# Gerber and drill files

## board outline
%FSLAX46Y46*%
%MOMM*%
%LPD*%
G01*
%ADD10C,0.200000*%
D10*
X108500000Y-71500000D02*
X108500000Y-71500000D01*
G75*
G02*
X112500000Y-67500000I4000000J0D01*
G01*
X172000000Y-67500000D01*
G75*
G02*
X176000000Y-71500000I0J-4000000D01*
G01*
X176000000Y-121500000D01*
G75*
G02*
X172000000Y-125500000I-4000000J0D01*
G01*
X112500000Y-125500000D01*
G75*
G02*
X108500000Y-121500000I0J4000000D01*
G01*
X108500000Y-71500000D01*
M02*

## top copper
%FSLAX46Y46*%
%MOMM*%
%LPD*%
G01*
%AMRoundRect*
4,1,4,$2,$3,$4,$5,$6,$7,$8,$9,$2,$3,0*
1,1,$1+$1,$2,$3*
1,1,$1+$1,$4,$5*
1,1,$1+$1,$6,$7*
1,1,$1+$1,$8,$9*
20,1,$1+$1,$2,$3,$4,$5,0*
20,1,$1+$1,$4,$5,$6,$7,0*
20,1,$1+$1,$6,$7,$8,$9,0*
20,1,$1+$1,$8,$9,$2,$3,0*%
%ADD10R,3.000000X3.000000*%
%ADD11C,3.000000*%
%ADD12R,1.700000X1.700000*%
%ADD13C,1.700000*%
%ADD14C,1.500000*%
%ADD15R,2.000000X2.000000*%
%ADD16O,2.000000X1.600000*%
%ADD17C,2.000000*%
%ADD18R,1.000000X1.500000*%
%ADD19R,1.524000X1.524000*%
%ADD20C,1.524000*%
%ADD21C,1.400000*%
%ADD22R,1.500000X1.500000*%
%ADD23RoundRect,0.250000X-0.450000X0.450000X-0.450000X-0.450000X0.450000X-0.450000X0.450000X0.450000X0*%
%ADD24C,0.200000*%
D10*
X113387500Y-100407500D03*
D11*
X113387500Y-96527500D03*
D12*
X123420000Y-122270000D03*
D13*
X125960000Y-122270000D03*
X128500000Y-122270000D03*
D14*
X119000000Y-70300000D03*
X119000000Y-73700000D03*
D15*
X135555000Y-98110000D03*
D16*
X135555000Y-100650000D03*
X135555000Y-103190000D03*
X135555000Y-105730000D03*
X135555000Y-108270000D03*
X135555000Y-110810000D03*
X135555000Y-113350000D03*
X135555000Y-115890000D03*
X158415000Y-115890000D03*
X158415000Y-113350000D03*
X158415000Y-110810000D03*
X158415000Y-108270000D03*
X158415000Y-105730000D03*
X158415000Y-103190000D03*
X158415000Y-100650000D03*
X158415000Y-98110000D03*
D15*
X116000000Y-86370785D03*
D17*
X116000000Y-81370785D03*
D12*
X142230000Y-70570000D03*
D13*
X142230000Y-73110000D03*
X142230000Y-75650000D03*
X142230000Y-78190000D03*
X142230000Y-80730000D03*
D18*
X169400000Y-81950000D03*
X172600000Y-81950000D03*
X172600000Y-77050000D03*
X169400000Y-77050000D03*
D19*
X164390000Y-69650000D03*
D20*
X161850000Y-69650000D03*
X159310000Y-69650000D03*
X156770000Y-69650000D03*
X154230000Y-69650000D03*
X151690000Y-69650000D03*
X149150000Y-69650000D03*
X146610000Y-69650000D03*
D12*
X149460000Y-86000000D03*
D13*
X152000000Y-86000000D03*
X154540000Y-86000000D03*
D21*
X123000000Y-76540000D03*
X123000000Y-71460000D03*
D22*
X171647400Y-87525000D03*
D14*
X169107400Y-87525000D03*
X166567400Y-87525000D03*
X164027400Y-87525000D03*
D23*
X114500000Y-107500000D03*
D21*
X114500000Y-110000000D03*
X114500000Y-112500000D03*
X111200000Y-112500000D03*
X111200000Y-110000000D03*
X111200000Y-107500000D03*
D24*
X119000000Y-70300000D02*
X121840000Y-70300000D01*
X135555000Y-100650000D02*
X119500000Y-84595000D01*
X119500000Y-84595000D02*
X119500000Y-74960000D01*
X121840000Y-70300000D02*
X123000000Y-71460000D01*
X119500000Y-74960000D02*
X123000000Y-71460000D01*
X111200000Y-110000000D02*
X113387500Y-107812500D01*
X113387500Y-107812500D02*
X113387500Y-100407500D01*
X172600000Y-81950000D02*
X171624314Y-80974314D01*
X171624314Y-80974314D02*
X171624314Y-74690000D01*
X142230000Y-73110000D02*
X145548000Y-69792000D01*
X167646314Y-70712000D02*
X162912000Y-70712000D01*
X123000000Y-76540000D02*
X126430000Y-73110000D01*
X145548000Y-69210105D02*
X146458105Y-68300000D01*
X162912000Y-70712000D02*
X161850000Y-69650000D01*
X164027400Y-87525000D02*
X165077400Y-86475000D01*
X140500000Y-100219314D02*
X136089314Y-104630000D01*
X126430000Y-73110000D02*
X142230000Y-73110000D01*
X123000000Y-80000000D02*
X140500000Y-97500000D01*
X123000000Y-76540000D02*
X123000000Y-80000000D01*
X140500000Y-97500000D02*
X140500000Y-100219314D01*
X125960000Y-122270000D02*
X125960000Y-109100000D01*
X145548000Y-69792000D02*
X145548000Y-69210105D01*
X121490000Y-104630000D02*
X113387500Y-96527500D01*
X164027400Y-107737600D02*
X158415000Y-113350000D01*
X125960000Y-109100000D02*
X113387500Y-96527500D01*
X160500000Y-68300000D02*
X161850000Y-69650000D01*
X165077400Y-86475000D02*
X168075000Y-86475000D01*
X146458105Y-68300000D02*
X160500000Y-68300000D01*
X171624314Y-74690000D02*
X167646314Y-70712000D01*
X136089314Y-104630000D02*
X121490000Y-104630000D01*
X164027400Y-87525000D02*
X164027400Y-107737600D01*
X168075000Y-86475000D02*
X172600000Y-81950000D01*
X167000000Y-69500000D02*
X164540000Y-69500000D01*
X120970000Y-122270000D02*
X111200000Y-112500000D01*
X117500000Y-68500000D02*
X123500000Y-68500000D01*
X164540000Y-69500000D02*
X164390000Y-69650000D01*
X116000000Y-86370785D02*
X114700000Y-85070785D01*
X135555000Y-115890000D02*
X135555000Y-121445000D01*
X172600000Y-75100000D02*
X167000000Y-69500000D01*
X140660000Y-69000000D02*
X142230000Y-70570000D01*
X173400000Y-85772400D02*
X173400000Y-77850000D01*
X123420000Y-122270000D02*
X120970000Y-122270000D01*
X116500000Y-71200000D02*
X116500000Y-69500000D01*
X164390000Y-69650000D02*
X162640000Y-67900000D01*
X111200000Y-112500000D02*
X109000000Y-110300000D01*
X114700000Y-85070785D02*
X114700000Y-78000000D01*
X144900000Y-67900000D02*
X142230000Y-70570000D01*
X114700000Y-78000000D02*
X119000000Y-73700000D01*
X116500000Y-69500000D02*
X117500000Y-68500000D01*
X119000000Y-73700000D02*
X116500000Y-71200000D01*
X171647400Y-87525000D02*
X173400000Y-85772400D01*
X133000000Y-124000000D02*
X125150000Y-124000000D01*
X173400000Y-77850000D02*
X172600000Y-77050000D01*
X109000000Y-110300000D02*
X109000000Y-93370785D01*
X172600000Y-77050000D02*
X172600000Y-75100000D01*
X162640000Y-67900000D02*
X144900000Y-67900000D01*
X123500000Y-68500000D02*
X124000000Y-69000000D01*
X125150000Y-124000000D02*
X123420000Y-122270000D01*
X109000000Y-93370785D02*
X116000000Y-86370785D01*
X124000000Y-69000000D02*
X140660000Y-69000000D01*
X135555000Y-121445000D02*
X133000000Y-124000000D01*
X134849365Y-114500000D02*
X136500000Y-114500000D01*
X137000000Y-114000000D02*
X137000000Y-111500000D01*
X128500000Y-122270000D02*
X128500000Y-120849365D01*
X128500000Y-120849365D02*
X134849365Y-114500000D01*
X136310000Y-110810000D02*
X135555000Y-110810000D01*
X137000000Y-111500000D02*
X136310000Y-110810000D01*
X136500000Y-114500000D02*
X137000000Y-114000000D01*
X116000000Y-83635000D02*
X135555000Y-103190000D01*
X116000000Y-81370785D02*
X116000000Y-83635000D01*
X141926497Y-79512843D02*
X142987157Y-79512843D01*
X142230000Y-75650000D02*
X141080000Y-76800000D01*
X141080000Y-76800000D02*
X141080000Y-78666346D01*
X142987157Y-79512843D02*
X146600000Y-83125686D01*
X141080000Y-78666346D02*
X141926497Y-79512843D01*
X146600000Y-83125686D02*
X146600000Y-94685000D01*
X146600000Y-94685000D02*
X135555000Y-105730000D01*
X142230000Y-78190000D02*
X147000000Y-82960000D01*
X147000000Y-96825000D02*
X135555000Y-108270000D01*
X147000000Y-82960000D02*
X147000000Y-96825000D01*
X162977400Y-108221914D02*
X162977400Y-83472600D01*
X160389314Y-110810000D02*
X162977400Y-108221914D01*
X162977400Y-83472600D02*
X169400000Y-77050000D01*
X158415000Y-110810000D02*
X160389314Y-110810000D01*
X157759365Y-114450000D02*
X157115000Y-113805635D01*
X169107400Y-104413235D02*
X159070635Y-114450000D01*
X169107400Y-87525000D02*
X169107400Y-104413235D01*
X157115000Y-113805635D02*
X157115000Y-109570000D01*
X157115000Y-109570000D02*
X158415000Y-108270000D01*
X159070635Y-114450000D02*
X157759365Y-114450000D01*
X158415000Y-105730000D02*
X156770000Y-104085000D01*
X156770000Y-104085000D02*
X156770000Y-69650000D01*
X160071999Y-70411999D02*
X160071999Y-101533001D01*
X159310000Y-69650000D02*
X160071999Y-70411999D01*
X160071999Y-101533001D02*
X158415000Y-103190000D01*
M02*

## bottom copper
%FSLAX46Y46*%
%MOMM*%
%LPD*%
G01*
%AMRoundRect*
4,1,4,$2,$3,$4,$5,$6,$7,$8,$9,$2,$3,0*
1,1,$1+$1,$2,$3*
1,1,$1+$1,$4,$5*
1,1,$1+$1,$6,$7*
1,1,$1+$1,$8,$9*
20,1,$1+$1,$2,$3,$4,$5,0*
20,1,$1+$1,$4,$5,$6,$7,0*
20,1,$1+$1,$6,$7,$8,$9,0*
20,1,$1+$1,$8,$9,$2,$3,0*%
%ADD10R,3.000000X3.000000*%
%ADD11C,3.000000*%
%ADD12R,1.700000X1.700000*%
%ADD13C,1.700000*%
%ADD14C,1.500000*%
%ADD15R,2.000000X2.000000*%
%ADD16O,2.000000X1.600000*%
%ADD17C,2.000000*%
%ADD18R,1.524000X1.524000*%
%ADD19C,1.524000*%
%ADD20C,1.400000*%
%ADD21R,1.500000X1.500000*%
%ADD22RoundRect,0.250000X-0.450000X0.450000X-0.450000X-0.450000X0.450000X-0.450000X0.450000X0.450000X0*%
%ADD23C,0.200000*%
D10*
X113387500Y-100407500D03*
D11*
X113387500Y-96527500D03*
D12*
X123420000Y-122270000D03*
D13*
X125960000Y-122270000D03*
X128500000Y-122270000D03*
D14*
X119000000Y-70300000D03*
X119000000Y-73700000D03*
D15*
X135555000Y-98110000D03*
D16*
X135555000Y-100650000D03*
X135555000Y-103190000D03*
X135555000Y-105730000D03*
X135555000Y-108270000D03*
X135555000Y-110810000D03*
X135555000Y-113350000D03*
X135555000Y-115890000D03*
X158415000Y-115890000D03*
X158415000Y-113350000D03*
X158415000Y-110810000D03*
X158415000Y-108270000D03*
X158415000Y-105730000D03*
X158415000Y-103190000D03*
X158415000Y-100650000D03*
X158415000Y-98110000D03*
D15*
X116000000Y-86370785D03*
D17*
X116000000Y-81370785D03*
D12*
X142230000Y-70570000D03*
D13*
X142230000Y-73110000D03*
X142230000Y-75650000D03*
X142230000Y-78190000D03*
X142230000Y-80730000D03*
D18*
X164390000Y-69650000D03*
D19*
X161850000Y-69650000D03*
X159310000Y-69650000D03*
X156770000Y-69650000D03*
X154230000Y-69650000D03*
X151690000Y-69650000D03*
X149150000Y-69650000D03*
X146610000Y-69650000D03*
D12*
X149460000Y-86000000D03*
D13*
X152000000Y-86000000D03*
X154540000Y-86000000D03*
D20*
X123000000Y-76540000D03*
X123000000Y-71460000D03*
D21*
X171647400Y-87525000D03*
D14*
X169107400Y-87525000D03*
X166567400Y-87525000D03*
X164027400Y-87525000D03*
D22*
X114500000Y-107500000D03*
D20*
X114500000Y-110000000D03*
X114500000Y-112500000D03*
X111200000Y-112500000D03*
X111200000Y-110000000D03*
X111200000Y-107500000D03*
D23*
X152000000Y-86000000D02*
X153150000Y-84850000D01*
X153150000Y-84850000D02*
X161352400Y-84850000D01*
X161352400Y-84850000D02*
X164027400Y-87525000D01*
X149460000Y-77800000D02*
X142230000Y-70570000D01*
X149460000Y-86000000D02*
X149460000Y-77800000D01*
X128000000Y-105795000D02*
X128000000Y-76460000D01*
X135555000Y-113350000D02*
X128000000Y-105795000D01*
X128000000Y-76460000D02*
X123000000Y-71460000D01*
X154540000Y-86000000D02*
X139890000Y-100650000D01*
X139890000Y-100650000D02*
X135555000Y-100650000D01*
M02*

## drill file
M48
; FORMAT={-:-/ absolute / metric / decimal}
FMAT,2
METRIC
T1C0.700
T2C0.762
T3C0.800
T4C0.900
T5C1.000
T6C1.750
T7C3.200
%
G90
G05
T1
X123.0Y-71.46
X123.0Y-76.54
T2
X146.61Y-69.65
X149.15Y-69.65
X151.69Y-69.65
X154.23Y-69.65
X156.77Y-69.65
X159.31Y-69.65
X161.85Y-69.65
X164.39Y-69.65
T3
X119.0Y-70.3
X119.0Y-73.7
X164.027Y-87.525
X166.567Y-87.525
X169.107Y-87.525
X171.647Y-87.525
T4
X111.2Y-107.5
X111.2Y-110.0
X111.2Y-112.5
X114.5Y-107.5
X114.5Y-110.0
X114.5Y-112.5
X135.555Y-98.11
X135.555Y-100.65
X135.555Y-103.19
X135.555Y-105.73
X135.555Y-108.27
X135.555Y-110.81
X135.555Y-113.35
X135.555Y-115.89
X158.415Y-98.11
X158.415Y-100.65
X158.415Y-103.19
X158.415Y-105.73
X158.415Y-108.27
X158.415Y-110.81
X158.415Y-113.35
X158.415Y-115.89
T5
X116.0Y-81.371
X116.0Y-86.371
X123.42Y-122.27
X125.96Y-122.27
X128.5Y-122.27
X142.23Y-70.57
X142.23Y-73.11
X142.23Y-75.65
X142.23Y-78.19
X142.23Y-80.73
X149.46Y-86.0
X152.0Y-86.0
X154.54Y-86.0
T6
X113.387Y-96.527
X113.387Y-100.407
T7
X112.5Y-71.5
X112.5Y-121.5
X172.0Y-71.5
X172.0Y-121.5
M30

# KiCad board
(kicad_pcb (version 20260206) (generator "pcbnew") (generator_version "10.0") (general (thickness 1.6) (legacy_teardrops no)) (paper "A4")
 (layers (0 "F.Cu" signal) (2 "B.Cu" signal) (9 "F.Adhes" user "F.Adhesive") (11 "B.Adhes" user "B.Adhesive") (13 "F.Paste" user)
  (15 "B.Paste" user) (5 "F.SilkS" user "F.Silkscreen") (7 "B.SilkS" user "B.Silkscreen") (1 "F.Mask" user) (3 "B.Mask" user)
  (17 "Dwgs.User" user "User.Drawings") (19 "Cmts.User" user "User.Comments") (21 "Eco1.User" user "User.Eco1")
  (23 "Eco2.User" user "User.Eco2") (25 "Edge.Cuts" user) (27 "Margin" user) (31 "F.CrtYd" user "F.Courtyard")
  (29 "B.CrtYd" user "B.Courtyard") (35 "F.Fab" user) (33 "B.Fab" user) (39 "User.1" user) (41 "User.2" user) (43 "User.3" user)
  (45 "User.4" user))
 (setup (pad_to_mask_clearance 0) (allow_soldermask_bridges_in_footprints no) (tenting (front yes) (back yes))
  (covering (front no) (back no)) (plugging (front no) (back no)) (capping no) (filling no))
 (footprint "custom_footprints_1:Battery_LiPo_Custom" (layer "F.Cu") (at 120.9375 98.0575 90)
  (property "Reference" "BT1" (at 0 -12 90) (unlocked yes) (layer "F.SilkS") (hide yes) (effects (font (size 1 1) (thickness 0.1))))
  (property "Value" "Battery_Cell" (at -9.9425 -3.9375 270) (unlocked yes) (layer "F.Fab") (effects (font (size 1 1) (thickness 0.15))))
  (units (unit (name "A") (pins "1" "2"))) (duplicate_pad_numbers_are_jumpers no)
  (pad "1" thru_hole rect (at -2.35 -7.55 90) (size 3 3) (drill 1.75) (layers "*.Cu" "*.Mask") (remove_unused_layers no) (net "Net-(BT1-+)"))
  (pad "2" thru_hole circle (at 1.53 -7.55 90) (size 3 3) (drill 1.75) (layers "*.Cu" "*.Mask") (remove_unused_layers no)
   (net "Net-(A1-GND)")))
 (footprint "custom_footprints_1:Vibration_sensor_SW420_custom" (layer "F.Cu") (at 130.27 122 90)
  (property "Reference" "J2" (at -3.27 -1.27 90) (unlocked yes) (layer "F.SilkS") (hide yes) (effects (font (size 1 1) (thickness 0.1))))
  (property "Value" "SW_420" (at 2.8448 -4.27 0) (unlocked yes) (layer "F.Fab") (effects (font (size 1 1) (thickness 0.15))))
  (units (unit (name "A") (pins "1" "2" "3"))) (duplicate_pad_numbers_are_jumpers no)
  (pad "1" thru_hole rect (at -0.27 -6.85 90) (size 1.7 1.7) (drill 1) (layers "*.Cu" "*.Mask") (remove_unused_layers no)
   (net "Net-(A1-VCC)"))
  (pad "2" thru_hole circle (at -0.27 -4.31 90) (size 1.7 1.7) (drill 1) (layers "*.Cu" "*.Mask") (remove_unused_layers no)
   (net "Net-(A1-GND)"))
  (pad "3" thru_hole circle (at -0.27 -1.77 90) (size 1.7 1.7) (drill 1) (layers "*.Cu" "*.Mask") (remove_unused_layers no)
   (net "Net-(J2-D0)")))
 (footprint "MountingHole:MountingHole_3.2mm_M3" (layer "F.Cu") (at 112.5 71.5 180)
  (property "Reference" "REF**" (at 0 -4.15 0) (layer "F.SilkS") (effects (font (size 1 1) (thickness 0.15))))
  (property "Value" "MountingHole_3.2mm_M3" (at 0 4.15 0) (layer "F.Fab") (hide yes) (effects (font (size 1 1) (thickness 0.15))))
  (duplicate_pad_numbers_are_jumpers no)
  (pad "" np_thru_hole circle (at 0 0 180) (size 3.2 3.2) (drill 3.2) (layers "*.Cu" "*.Mask")))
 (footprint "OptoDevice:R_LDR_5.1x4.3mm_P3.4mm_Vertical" (layer "F.Cu") (at 119 70.3 -90)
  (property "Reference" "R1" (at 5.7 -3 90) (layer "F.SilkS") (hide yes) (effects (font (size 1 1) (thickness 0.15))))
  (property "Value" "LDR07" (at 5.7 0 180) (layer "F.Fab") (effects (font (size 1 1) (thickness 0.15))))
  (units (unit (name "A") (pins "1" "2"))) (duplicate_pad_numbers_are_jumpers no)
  (pad "1" thru_hole circle (at 0 0 270) (size 1.5 1.5) (drill 0.8) (layers "*.Cu" "*.Mask") (remove_unused_layers no)
   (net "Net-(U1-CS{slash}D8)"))
  (pad "2" thru_hole circle (at 3.4 0 270) (size 1.5 1.5) (drill 0.8) (layers "*.Cu" "*.Mask") (remove_unused_layers no)
   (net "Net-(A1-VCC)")))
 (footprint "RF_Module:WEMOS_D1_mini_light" (layer "F.Cu") (at 135.555 98.11)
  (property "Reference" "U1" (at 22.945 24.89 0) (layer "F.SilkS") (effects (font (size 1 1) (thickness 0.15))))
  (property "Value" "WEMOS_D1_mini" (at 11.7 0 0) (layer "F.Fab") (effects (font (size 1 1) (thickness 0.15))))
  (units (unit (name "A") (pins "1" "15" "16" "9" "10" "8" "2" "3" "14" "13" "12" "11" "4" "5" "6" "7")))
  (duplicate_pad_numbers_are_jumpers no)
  (pad "1" thru_hole rect (at 0 0) (size 2 2) (drill 0.9) (layers "*.Cu" "*.Mask") (remove_unused_layers no)
   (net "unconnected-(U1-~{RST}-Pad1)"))
  (pad "2" thru_hole oval (at 0 2.54) (size 2 1.6) (drill 0.9) (layers "*.Cu" "*.Mask") (remove_unused_layers no) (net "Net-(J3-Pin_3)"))
  (pad "3" thru_hole oval (at 0 5.08) (size 2 1.6) (drill 0.9) (layers "*.Cu" "*.Mask") (remove_unused_layers no) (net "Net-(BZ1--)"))
  (pad "4" thru_hole oval (at 0 7.62) (size 2 1.6) (drill 0.9) (layers "*.Cu" "*.Mask") (remove_unused_layers no) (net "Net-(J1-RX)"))
  (pad "5" thru_hole oval (at 0 10.16) (size 2 1.6) (drill 0.9) (layers "*.Cu" "*.Mask") (remove_unused_layers no) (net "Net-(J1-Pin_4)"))
  (pad "6" thru_hole oval (at 0 12.7) (size 2 1.6) (drill 0.9) (layers "*.Cu" "*.Mask") (remove_unused_layers no) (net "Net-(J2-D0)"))
  (pad "7" thru_hole oval (at 0 15.24) (size 2 1.6) (drill 0.9) (layers "*.Cu" "*.Mask") (remove_unused_layers no)
   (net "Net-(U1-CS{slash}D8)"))
  (pad "8" thru_hole oval (at 0 17.78) (size 2 1.6) (drill 0.9) (layers "*.Cu" "*.Mask") (remove_unused_layers no) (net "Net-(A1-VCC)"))
  (pad "9" thru_hole oval (at 22.86 17.78) (size 2 1.6) (drill 0.9) (layers "*.Cu" "*.Mask") (remove_unused_layers no)
   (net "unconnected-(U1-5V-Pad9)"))
  (pad "10" thru_hole oval (at 22.86 15.24) (size 2 1.6) (drill 0.9) (layers "*.Cu" "*.Mask") (remove_unused_layers no) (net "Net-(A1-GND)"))
  (pad "11" thru_hole oval (at 22.86 12.7) (size 2 1.6) (drill 0.9) (layers "*.Cu" "*.Mask") (remove_unused_layers no) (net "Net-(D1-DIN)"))
  (pad "12" thru_hole oval (at 22.86 10.16) (size 2 1.6) (drill 0.9) (layers "*.Cu" "*.Mask") (remove_unused_layers no) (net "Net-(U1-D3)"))
  (pad "13" thru_hole oval (at 22.86 7.62) (size 2 1.6) (drill 0.9) (layers "*.Cu" "*.Mask") (remove_unused_layers no) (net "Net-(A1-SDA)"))
  (pad "14" thru_hole oval (at 22.86 5.08) (size 2 1.6) (drill 0.9) (layers "*.Cu" "*.Mask") (remove_unused_layers no) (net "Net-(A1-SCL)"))
  (pad "15" thru_hole oval (at 22.86 2.54) (size 2 1.6) (drill 0.9) (layers "*.Cu" "*.Mask") (remove_unused_layers no)
   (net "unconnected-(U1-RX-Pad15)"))
  (pad "16" thru_hole oval (at 22.86 0) (size 2 1.6) (drill 0.9) (layers "*.Cu" "*.Mask") (remove_unused_layers no)
   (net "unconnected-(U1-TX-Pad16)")))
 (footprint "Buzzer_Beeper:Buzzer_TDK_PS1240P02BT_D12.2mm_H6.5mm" (layer "F.Cu") (at 116 86.370785 90)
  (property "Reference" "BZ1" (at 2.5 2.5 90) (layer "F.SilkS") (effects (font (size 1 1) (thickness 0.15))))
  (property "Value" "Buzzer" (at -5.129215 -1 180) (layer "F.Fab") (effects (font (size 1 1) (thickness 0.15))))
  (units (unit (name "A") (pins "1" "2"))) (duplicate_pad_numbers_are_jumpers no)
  (pad "1" thru_hole rect (at 0 0 90) (size 2 2) (drill 1) (layers "*.Cu" "*.Mask") (remove_unused_layers no) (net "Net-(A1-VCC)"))
  (pad "2" thru_hole circle (at 5 0 90) (size 2 2) (drill 1) (layers "*.Cu" "*.Mask") (remove_unused_layers no) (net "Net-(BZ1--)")))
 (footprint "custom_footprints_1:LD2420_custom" (layer "F.Cu") (at 134.73 77.57)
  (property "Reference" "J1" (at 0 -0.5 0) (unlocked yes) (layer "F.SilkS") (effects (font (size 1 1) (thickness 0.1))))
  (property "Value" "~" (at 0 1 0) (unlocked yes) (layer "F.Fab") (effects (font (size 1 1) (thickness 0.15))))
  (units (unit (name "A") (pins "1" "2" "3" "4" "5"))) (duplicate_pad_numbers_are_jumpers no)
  (pad "1" thru_hole rect (at 7.5 -7) (size 1.7 1.7) (drill 1) (layers "*.Cu" "*.Mask") (remove_unused_layers no) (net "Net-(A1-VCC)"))
  (pad "2" thru_hole circle (at 7.5 -4.46) (size 1.7 1.7) (drill 1) (layers "*.Cu" "*.Mask") (remove_unused_layers no) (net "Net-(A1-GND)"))
  (pad "3" thru_hole circle (at 7.5 -1.92) (size 1.7 1.7) (drill 1) (layers "*.Cu" "*.Mask") (remove_unused_layers no) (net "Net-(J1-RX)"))
  (pad "4" thru_hole circle (at 7.5 0.62) (size 1.7 1.7) (drill 1) (layers "*.Cu" "*.Mask") (remove_unused_layers no) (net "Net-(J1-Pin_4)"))
  (pad "5" thru_hole circle (at 7.5 3.16) (size 1.7 1.7) (drill 1) (layers "*.Cu" "*.Mask") (remove_unused_layers no)
   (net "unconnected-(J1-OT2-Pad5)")))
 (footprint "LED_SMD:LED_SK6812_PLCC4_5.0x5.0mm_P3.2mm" (layer "F.Cu") (at 171 79.5 90)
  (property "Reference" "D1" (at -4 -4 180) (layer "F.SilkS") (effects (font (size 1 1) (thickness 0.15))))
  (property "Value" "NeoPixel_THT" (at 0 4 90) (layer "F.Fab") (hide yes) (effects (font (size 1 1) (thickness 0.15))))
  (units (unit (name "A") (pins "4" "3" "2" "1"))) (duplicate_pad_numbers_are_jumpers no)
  (pad "1" smd rect (at -2.45 -1.6 270) (size 1.5 1) (layers "F.Cu" "F.Mask" "F.Paste") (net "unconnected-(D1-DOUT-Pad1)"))
  (pad "2" smd rect (at -2.45 1.6 270) (size 1.5 1) (layers "F.Cu" "F.Mask" "F.Paste") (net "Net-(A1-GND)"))
  (pad "3" smd rect (at 2.45 1.6 270) (size 1.5 1) (layers "F.Cu" "F.Mask" "F.Paste") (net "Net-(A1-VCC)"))
  (pad "4" smd rect (at 2.45 -1.6 270) (size 1.5 1) (layers "F.Cu" "F.Mask" "F.Paste") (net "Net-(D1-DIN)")))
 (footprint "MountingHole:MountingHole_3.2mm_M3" (layer "F.Cu") (at 172 71.5 180)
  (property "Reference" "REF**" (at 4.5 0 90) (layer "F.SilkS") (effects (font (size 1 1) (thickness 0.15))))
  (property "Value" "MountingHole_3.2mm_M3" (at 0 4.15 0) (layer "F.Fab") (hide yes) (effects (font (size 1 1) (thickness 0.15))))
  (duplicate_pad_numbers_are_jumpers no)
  (pad "" np_thru_hole circle (at 0 0 180) (size 3.2 3.2) (drill 3.2) (layers "*.Cu" "*.Mask")))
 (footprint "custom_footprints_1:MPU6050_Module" (layer "F.Cu") (at 164.39 69.65 -90)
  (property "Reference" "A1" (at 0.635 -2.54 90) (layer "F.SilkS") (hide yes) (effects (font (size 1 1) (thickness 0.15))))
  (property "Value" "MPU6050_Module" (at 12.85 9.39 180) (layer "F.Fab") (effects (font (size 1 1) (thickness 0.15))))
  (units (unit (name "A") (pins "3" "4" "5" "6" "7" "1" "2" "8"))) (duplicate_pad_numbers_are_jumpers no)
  (pad "1" thru_hole rect (at 0 0 270) (size 1.524 1.524) (drill 0.762) (layers "*.Cu" "*.Mask") (remove_unused_layers no)
   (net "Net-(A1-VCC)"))
  (pad "2" thru_hole circle (at 0 2.54 270) (size 1.524 1.524) (drill 0.762) (layers "*.Cu" "*.Mask") (remove_unused_layers no)
   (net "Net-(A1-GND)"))
  (pad "3" thru_hole circle (at 0 5.08 270) (size 1.524 1.524) (drill 0.762) (layers "*.Cu" "*.Mask") (remove_unused_layers no)
   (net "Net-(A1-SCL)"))
  (pad "4" thru_hole circle (at 0 7.62 270) (size 1.524 1.524) (drill 0.762) (layers "*.Cu" "*.Mask") (remove_unused_layers no)
   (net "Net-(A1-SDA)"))
  (pad "5" thru_hole circle (at 0 10.16 270) (size 1.524 1.524) (drill 0.762) (layers "*.Cu" "*.Mask") (remove_unused_layers no)
   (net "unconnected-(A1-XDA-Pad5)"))
  (pad "6" thru_hole circle (at 0 12.7 270) (size 1.524 1.524) (drill 0.762) (layers "*.Cu" "*.Mask") (remove_unused_layers no)
   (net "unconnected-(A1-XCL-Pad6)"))
  (pad "7" thru_hole circle (at 0 15.24 270) (size 1.524 1.524) (drill 0.762) (layers "*.Cu" "*.Mask") (remove_unused_layers no)
   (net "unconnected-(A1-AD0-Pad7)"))
  (pad "8" thru_hole circle (at 0 17.78 270) (size 1.524 1.524) (drill 0.762) (layers "*.Cu" "*.Mask") (remove_unused_layers no)
   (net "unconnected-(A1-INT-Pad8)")))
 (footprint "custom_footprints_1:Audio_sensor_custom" (layer "F.Cu") (at 155.048 86.0588 90)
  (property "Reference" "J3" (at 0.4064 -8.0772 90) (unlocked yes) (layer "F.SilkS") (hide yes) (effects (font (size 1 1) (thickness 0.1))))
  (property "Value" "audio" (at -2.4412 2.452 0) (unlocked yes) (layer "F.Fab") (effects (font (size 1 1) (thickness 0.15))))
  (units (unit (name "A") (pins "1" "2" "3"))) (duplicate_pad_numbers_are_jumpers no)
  (pad "1" thru_hole rect (at 0.0588 -5.588 90) (size 1.7 1.7) (drill 1) (layers "*.Cu" "*.Mask") (remove_unused_layers no)
   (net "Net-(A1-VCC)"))
  (pad "2" thru_hole circle (at 0.0588 -3.048 90) (size 1.7 1.7) (drill 1) (layers "*.Cu" "*.Mask") (remove_unused_layers no)
   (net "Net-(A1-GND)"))
  (pad "3" thru_hole circle (at 0.0588 -0.508 90) (size 1.7 1.7) (drill 1) (layers "*.Cu" "*.Mask") (remove_unused_layers no)
   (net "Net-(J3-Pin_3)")))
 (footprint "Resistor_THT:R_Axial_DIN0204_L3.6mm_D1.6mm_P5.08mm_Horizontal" (layer "F.Cu") (at 123 76.54 90)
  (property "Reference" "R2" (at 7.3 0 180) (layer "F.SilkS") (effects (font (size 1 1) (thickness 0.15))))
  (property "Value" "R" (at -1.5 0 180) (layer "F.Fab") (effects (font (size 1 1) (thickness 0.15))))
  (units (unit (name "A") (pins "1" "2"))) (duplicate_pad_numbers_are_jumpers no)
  (pad "1" thru_hole circle (at 0 0 90) (size 1.4 1.4) (drill 0.7) (layers "*.Cu" "*.Mask") (remove_unused_layers no) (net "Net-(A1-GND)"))
  (pad "2" thru_hole circle (at 5.08 0 90) (size 1.4 1.4) (drill 0.7) (layers "*.Cu" "*.Mask") (remove_unused_layers no)
   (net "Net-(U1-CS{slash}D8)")))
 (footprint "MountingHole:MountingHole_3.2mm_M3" (layer "F.Cu") (at 112.5 121.5)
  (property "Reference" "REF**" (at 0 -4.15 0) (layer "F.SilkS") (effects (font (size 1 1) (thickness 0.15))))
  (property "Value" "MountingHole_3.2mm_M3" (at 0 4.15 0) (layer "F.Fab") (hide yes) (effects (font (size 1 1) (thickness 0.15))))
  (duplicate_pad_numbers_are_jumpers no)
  (pad "" np_thru_hole circle (at 0 0) (size 3.2 3.2) (drill 3.2) (layers "*.Cu" "*.Mask")))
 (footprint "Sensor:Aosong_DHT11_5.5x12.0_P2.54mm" (layer "F.Cu") (at 171.6474 87.525 -90)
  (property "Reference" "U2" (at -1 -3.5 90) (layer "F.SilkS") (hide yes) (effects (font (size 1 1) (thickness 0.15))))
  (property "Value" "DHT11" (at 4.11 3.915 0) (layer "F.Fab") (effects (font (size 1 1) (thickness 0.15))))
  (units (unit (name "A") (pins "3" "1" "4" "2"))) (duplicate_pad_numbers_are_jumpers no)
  (pad "1" thru_hole rect (at 0 0 270) (size 1.5 1.5) (drill 0.8) (layers "*.Cu" "*.Mask") (remove_unused_layers no) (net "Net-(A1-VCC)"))
  (pad "2" thru_hole circle (at 0 2.54 270) (size 1.5 1.5) (drill 0.8) (layers "*.Cu" "*.Mask") (remove_unused_layers no)
   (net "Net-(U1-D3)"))
  (pad "3" thru_hole circle (at 0 5.08 270) (size 1.5 1.5) (drill 0.8) (layers "*.Cu" "*.Mask") (remove_unused_layers no)
   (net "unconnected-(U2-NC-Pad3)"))
  (pad "4" thru_hole circle (at 0 7.62 270) (size 1.5 1.5) (drill 0.8) (layers "*.Cu" "*.Mask") (remove_unused_layers no)
   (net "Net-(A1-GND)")))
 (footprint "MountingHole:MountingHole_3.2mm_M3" (layer "F.Cu") (at 172 121.5)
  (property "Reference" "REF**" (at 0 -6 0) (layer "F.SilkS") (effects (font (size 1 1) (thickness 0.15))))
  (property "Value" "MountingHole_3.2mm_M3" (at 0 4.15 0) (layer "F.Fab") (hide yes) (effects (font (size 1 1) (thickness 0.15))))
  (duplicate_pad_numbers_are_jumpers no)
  (pad "" np_thru_hole circle (at 0 0) (size 3.2 3.2) (drill 3.2) (layers "*.Cu" "*.Mask")))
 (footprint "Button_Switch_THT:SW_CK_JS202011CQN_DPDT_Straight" (layer "F.Cu") (at 114.5 107.5 -90)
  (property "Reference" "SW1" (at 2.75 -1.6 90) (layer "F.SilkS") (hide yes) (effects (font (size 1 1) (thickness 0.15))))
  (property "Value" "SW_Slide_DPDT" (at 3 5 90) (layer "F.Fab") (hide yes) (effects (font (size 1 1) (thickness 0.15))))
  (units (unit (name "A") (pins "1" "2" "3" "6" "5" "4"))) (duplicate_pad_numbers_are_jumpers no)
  (pad "1" thru_hole roundrect (at 0 0 270) (size 1.4 1.4) (drill 0.9) (layers "*.Cu" "*.Mask") (remove_unused_layers no)
   (roundrect_rratio 0.1785714286) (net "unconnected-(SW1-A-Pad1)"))
  (pad "2" thru_hole circle (at 2.5 0 270) (size 1.4 1.4) (drill 0.9) (layers "*.Cu" "*.Mask") (remove_unused_layers no)
   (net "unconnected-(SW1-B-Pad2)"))
  (pad "3" thru_hole circle (at 5 0 270) (size 1.4 1.4) (drill 0.9) (layers "*.Cu" "*.Mask") (remove_unused_layers no)
   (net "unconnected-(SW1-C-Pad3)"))
  (pad "4" thru_hole circle (at 5 3.3 270) (size 1.4 1.4) (drill 0.9) (layers "*.Cu" "*.Mask") (remove_unused_layers no)
   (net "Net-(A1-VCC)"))
  (pad "5" thru_hole circle (at 2.5 3.3 270) (size 1.4 1.4) (drill 0.9) (layers "*.Cu" "*.Mask") (remove_unused_layers no)
   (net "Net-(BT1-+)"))
  (pad "6" thru_hole circle (at 0 3.3 270) (size 1.4 1.4) (drill 0.9) (layers "*.Cu" "*.Mask") (remove_unused_layers no)
   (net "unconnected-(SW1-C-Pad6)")))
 (gr_rect (start 108.5 67.5) (end 176 125.5) (radius 4) (stroke (width 0.2) (type default)) (fill no) (layer "Edge.Cuts"))
 (segment (start 119 70.3) (end 121.84 70.3) (width 0.2) (layer "F.Cu") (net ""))
 (segment (start 135.555 100.65) (end 119.5 84.595) (width 0.2) (layer "F.Cu") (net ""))
 (segment (start 119.5 84.595) (end 119.5 74.96) (width 0.2) (layer "F.Cu") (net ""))
 (segment (start 121.84 70.3) (end 123 71.46) (width 0.2) (layer "F.Cu") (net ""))
 (segment (start 119.5 74.96) (end 123 71.46) (width 0.2) (layer "F.Cu") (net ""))
 (segment (start 111.2 110) (end 113.3875 107.8125) (width 0.2) (layer "F.Cu") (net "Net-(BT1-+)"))
 (segment (start 113.3875 107.8125) (end 113.3875 100.4075) (width 0.2) (layer "F.Cu") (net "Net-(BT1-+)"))
 (segment (start 172.6 81.95) (end 171.624314 80.974314) (width 0.2) (layer "F.Cu") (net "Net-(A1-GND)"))
 (segment (start 171.624314 80.974314) (end 171.624314 74.69) (width 0.2) (layer "F.Cu") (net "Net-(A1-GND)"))
 (segment (start 142.23 73.11) (end 145.548 69.792) (width 0.2) (layer "F.Cu") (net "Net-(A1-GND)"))
 (segment (start 167.646314 70.712) (end 162.912 70.712) (width 0.2) (layer "F.Cu") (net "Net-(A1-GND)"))
 (segment (start 123 76.54) (end 126.43 73.11) (width 0.2) (layer "F.Cu") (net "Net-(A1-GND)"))
 (segment (start 145.548 69.210105) (end 146.458105 68.3) (width 0.2) (layer "F.Cu") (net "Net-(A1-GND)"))
 (segment (start 162.912 70.712) (end 161.85 69.65) (width 0.2) (layer "F.Cu") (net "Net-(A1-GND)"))
 (segment (start 164.0274 87.525) (end 165.0774 86.475) (width 0.2) (layer "F.Cu") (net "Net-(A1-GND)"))
 (segment (start 140.5 100.219314) (end 136.089314 104.63) (width 0.2) (layer "F.Cu") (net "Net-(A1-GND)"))
 (segment (start 126.43 73.11) (end 142.23 73.11) (width 0.2) (layer "F.Cu") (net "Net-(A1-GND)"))
 (segment (start 123 80) (end 140.5 97.5) (width 0.2) (layer "F.Cu") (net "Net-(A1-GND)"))
 (segment (start 123 76.54) (end 123 80) (width 0.2) (layer "F.Cu") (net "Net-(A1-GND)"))
 (segment (start 140.5 97.5) (end 140.5 100.219314) (width 0.2) (layer "F.Cu") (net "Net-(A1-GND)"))
 (segment (start 125.96 122.27) (end 125.96 109.1) (width 0.2) (layer "F.Cu") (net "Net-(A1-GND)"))
 (segment (start 145.548 69.792) (end 145.548 69.210105) (width 0.2) (layer "F.Cu") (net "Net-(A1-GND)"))
 (segment (start 121.49 104.63) (end 113.3875 96.5275) (width 0.2) (layer "F.Cu") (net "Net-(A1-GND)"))
 (segment (start 164.0274 107.7376) (end 158.415 113.35) (width 0.2) (layer "F.Cu") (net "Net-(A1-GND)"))
 (segment (start 125.96 109.1) (end 113.3875 96.5275) (width 0.2) (layer "F.Cu") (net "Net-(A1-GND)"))
 (segment (start 160.5 68.3) (end 161.85 69.65) (width 0.2) (layer "F.Cu") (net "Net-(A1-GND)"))
 (segment (start 165.0774 86.475) (end 168.075 86.475) (width 0.2) (layer "F.Cu") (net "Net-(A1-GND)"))
 (segment (start 146.458105 68.3) (end 160.5 68.3) (width 0.2) (layer "F.Cu") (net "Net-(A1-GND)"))
 (segment (start 171.624314 74.69) (end 167.646314 70.712) (width 0.2) (layer "F.Cu") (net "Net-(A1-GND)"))
 (segment (start 136.089314 104.63) (end 121.49 104.63) (width 0.2) (layer "F.Cu") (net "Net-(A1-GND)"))
 (segment (start 164.0274 87.525) (end 164.0274 107.7376) (width 0.2) (layer "F.Cu") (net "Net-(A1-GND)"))
 (segment (start 168.075 86.475) (end 172.6 81.95) (width 0.2) (layer "F.Cu") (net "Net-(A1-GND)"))
 (segment (start 152 86) (end 153.15 84.85) (width 0.2) (layer "B.Cu") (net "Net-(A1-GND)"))
 (segment (start 153.15 84.85) (end 161.3524 84.85) (width 0.2) (layer "B.Cu") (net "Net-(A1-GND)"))
 (segment (start 161.3524 84.85) (end 164.0274 87.525) (width 0.2) (layer "B.Cu") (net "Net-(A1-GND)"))
 (segment (start 167 69.5) (end 164.54 69.5) (width 0.2) (layer "F.Cu") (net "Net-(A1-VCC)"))
 (segment (start 120.97 122.27) (end 111.2 112.5) (width 0.2) (layer "F.Cu") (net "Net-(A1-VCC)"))
 (segment (start 117.5 68.5) (end 123.5 68.5) (width 0.2) (layer "F.Cu") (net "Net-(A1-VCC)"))
 (segment (start 164.54 69.5) (end 164.39 69.65) (width 0.2) (layer "F.Cu") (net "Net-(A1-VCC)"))
 (segment (start 116 86.370785) (end 114.7 85.070785) (width 0.2) (layer "F.Cu") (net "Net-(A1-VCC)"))
 (segment (start 135.555 115.89) (end 135.555 121.445) (width 0.2) (layer "F.Cu") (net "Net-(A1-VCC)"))
 (segment (start 172.6 75.1) (end 167 69.5) (width 0.2) (layer "F.Cu") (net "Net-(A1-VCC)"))
 (segment (start 140.66 69) (end 142.23 70.57) (width 0.2) (layer "F.Cu") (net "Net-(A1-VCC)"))
 (segment (start 173.4 85.7724) (end 173.4 77.85) (width 0.2) (layer "F.Cu") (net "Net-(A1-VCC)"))
 (segment (start 123.42 122.27) (end 120.97 122.27) (width 0.2) (layer "F.Cu") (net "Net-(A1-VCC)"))
 (segment (start 116.5 71.2) (end 116.5 69.5) (width 0.2) (layer "F.Cu") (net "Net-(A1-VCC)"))
 (segment (start 164.39 69.65) (end 162.64 67.9) (width 0.2) (layer "F.Cu") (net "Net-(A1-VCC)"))
 (segment (start 111.2 112.5) (end 109 110.3) (width 0.2) (layer "F.Cu") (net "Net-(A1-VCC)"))
 (segment (start 114.7 85.070785) (end 114.7 78) (width 0.2) (layer "F.Cu") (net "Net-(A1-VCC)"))
 (segment (start 144.9 67.9) (end 142.23 70.57) (width 0.2) (layer "F.Cu") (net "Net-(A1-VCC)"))
 (segment (start 114.7 78) (end 119 73.7) (width 0.2) (layer "F.Cu") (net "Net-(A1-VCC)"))
 (segment (start 116.5 69.5) (end 117.5 68.5) (width 0.2) (layer "F.Cu") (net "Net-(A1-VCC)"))
 (segment (start 119 73.7) (end 116.5 71.2) (width 0.2) (layer "F.Cu") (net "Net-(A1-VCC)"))
 (segment (start 171.6474 87.525) (end 173.4 85.7724) (width 0.2) (layer "F.Cu") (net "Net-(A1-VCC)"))
 (segment (start 133 124) (end 125.15 124) (width 0.2) (layer "F.Cu") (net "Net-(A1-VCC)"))
 (segment (start 173.4 77.85) (end 172.6 77.05) (width 0.2) (layer "F.Cu") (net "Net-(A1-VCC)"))
 (segment (start 109 110.3) (end 109 93.370785) (width 0.2) (layer "F.Cu") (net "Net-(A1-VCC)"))
 (segment (start 172.6 77.05) (end 172.6 75.1) (width 0.2) (layer "F.Cu") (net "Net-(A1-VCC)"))
 (segment (start 162.64 67.9) (end 144.9 67.9) (width 0.2) (layer "F.Cu") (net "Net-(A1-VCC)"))
 (segment (start 123.5 68.5) (end 124 69) (width 0.2) (layer "F.Cu") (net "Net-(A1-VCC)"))
 (segment (start 125.15 124) (end 123.42 122.27) (width 0.2) (layer "F.Cu") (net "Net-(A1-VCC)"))
 (segment (start 109 93.370785) (end 116 86.370785) (width 0.2) (layer "F.Cu") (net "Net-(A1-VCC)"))
 (segment (start 124 69) (end 140.66 69) (width 0.2) (layer "F.Cu") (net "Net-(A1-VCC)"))
 (segment (start 135.555 121.445) (end 133 124) (width 0.2) (layer "F.Cu") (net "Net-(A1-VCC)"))
 (segment (start 149.46 77.8) (end 142.23 70.57) (width 0.2) (layer "B.Cu") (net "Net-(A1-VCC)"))
 (segment (start 149.46 86) (end 149.46 77.8) (width 0.2) (layer "B.Cu") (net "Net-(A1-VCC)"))
 (segment (start 134.849365 114.5) (end 136.5 114.5) (width 0.2) (layer "F.Cu") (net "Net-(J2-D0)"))
 (segment (start 137 114) (end 137 111.5) (width 0.2) (layer "F.Cu") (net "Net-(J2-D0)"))
 (segment (start 128.5 122.27) (end 128.5 120.849365) (width 0.2) (layer "F.Cu") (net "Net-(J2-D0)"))
 (segment (start 128.5 120.849365) (end 134.849365 114.5) (width 0.2) (layer "F.Cu") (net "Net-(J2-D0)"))
 (segment (start 136.31 110.81) (end 135.555 110.81) (width 0.2) (layer "F.Cu") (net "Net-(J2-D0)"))
 (segment (start 137 111.5) (end 136.31 110.81) (width 0.2) (layer "F.Cu") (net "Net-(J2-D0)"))
 (segment (start 136.5 114.5) (end 137 114) (width 0.2) (layer "F.Cu") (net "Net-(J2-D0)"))
 (segment (start 128 105.795) (end 128 76.46) (width 0.2) (layer "B.Cu") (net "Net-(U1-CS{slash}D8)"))
 (segment (start 135.555 113.35) (end 128 105.795) (width 0.2) (layer "B.Cu") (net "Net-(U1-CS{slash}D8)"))
 (segment (start 128 76.46) (end 123 71.46) (width 0.2) (layer "B.Cu") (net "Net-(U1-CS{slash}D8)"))
 (segment (start 154.54 86) (end 139.89 100.65) (width 0.2) (layer "B.Cu") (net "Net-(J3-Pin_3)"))
 (segment (start 139.89 100.65) (end 135.555 100.65) (width 0.2) (layer "B.Cu") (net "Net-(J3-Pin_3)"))
 (segment (start 116 83.635) (end 135.555 103.19) (width 0.2) (layer "F.Cu") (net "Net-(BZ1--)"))
 (segment (start 116 81.370785) (end 116 83.635) (width 0.2) (layer "F.Cu") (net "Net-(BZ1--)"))
 (segment (start 141.926497 79.512843) (end 142.987157 79.512843) (width 0.2) (layer "F.Cu") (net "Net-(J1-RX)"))
 (segment (start 142.23 75.65) (end 141.08 76.8) (width 0.2) (layer "F.Cu") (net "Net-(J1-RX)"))
 (segment (start 141.08 76.8) (end 141.08 78.666346) (width 0.2) (layer "F.Cu") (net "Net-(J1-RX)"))
 (segment (start 142.987157 79.512843) (end 146.6 83.125686) (width 0.2) (layer "F.Cu") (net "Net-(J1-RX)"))
 (segment (start 141.08 78.666346) (end 141.926497 79.512843) (width 0.2) (layer "F.Cu") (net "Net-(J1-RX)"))
 (segment (start 146.6 83.125686) (end 146.6 94.685) (width 0.2) (layer "F.Cu") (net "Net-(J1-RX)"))
 (segment (start 146.6 94.685) (end 135.555 105.73) (width 0.2) (layer "F.Cu") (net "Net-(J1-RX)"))
 (segment (start 142.23 78.19) (end 147 82.96) (width 0.2) (layer "F.Cu") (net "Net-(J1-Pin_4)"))
 (segment (start 147 96.825) (end 135.555 108.27) (width 0.2) (layer "F.Cu") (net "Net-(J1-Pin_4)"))
 (segment (start 147 82.96) (end 147 96.825) (width 0.2) (layer "F.Cu") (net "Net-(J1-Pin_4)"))
 (segment (start 162.9774 108.221914) (end 162.9774 83.4726) (width 0.2) (layer "F.Cu") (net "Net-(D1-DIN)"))
 (segment (start 160.389314 110.81) (end 162.9774 108.221914) (width 0.2) (layer "F.Cu") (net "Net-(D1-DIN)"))
 (segment (start 162.9774 83.4726) (end 169.4 77.05) (width 0.2) (layer "F.Cu") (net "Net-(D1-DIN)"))
 (segment (start 158.415 110.81) (end 160.389314 110.81) (width 0.2) (layer "F.Cu") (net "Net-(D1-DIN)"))
 (segment (start 157.759365 114.45) (end 157.115 113.805635) (width 0.2) (layer "F.Cu") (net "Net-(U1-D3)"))
 (segment (start 169.1074 104.413235) (end 159.070635 114.45) (width 0.2) (layer "F.Cu") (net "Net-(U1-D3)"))
 (segment (start 169.1074 87.525) (end 169.1074 104.413235) (width 0.2) (layer "F.Cu") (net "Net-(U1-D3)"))
 (segment (start 157.115 113.805635) (end 157.115 109.57) (width 0.2) (layer "F.Cu") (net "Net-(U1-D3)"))
 (segment (start 157.115 109.57) (end 158.415 108.27) (width 0.2) (layer "F.Cu") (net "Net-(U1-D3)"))
 (segment (start 159.070635 114.45) (end 157.759365 114.45) (width 0.2) (layer "F.Cu") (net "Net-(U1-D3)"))
 (segment (start 158.415 105.73) (end 156.77 104.085) (width 0.2) (layer "F.Cu") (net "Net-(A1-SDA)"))
 (segment (start 156.77 104.085) (end 156.77 69.65) (width 0.2) (layer "F.Cu") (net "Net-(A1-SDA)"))
 (segment (start 160.071999 70.411999) (end 160.071999 101.533001) (width 0.2) (layer "F.Cu") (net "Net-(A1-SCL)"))
 (segment (start 159.31 69.65) (end 160.071999 70.411999) (width 0.2) (layer "F.Cu") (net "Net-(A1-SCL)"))
 (segment (start 160.071999 101.533001) (end 158.415 103.19) (width 0.2) (layer "F.Cu") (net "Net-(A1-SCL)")))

